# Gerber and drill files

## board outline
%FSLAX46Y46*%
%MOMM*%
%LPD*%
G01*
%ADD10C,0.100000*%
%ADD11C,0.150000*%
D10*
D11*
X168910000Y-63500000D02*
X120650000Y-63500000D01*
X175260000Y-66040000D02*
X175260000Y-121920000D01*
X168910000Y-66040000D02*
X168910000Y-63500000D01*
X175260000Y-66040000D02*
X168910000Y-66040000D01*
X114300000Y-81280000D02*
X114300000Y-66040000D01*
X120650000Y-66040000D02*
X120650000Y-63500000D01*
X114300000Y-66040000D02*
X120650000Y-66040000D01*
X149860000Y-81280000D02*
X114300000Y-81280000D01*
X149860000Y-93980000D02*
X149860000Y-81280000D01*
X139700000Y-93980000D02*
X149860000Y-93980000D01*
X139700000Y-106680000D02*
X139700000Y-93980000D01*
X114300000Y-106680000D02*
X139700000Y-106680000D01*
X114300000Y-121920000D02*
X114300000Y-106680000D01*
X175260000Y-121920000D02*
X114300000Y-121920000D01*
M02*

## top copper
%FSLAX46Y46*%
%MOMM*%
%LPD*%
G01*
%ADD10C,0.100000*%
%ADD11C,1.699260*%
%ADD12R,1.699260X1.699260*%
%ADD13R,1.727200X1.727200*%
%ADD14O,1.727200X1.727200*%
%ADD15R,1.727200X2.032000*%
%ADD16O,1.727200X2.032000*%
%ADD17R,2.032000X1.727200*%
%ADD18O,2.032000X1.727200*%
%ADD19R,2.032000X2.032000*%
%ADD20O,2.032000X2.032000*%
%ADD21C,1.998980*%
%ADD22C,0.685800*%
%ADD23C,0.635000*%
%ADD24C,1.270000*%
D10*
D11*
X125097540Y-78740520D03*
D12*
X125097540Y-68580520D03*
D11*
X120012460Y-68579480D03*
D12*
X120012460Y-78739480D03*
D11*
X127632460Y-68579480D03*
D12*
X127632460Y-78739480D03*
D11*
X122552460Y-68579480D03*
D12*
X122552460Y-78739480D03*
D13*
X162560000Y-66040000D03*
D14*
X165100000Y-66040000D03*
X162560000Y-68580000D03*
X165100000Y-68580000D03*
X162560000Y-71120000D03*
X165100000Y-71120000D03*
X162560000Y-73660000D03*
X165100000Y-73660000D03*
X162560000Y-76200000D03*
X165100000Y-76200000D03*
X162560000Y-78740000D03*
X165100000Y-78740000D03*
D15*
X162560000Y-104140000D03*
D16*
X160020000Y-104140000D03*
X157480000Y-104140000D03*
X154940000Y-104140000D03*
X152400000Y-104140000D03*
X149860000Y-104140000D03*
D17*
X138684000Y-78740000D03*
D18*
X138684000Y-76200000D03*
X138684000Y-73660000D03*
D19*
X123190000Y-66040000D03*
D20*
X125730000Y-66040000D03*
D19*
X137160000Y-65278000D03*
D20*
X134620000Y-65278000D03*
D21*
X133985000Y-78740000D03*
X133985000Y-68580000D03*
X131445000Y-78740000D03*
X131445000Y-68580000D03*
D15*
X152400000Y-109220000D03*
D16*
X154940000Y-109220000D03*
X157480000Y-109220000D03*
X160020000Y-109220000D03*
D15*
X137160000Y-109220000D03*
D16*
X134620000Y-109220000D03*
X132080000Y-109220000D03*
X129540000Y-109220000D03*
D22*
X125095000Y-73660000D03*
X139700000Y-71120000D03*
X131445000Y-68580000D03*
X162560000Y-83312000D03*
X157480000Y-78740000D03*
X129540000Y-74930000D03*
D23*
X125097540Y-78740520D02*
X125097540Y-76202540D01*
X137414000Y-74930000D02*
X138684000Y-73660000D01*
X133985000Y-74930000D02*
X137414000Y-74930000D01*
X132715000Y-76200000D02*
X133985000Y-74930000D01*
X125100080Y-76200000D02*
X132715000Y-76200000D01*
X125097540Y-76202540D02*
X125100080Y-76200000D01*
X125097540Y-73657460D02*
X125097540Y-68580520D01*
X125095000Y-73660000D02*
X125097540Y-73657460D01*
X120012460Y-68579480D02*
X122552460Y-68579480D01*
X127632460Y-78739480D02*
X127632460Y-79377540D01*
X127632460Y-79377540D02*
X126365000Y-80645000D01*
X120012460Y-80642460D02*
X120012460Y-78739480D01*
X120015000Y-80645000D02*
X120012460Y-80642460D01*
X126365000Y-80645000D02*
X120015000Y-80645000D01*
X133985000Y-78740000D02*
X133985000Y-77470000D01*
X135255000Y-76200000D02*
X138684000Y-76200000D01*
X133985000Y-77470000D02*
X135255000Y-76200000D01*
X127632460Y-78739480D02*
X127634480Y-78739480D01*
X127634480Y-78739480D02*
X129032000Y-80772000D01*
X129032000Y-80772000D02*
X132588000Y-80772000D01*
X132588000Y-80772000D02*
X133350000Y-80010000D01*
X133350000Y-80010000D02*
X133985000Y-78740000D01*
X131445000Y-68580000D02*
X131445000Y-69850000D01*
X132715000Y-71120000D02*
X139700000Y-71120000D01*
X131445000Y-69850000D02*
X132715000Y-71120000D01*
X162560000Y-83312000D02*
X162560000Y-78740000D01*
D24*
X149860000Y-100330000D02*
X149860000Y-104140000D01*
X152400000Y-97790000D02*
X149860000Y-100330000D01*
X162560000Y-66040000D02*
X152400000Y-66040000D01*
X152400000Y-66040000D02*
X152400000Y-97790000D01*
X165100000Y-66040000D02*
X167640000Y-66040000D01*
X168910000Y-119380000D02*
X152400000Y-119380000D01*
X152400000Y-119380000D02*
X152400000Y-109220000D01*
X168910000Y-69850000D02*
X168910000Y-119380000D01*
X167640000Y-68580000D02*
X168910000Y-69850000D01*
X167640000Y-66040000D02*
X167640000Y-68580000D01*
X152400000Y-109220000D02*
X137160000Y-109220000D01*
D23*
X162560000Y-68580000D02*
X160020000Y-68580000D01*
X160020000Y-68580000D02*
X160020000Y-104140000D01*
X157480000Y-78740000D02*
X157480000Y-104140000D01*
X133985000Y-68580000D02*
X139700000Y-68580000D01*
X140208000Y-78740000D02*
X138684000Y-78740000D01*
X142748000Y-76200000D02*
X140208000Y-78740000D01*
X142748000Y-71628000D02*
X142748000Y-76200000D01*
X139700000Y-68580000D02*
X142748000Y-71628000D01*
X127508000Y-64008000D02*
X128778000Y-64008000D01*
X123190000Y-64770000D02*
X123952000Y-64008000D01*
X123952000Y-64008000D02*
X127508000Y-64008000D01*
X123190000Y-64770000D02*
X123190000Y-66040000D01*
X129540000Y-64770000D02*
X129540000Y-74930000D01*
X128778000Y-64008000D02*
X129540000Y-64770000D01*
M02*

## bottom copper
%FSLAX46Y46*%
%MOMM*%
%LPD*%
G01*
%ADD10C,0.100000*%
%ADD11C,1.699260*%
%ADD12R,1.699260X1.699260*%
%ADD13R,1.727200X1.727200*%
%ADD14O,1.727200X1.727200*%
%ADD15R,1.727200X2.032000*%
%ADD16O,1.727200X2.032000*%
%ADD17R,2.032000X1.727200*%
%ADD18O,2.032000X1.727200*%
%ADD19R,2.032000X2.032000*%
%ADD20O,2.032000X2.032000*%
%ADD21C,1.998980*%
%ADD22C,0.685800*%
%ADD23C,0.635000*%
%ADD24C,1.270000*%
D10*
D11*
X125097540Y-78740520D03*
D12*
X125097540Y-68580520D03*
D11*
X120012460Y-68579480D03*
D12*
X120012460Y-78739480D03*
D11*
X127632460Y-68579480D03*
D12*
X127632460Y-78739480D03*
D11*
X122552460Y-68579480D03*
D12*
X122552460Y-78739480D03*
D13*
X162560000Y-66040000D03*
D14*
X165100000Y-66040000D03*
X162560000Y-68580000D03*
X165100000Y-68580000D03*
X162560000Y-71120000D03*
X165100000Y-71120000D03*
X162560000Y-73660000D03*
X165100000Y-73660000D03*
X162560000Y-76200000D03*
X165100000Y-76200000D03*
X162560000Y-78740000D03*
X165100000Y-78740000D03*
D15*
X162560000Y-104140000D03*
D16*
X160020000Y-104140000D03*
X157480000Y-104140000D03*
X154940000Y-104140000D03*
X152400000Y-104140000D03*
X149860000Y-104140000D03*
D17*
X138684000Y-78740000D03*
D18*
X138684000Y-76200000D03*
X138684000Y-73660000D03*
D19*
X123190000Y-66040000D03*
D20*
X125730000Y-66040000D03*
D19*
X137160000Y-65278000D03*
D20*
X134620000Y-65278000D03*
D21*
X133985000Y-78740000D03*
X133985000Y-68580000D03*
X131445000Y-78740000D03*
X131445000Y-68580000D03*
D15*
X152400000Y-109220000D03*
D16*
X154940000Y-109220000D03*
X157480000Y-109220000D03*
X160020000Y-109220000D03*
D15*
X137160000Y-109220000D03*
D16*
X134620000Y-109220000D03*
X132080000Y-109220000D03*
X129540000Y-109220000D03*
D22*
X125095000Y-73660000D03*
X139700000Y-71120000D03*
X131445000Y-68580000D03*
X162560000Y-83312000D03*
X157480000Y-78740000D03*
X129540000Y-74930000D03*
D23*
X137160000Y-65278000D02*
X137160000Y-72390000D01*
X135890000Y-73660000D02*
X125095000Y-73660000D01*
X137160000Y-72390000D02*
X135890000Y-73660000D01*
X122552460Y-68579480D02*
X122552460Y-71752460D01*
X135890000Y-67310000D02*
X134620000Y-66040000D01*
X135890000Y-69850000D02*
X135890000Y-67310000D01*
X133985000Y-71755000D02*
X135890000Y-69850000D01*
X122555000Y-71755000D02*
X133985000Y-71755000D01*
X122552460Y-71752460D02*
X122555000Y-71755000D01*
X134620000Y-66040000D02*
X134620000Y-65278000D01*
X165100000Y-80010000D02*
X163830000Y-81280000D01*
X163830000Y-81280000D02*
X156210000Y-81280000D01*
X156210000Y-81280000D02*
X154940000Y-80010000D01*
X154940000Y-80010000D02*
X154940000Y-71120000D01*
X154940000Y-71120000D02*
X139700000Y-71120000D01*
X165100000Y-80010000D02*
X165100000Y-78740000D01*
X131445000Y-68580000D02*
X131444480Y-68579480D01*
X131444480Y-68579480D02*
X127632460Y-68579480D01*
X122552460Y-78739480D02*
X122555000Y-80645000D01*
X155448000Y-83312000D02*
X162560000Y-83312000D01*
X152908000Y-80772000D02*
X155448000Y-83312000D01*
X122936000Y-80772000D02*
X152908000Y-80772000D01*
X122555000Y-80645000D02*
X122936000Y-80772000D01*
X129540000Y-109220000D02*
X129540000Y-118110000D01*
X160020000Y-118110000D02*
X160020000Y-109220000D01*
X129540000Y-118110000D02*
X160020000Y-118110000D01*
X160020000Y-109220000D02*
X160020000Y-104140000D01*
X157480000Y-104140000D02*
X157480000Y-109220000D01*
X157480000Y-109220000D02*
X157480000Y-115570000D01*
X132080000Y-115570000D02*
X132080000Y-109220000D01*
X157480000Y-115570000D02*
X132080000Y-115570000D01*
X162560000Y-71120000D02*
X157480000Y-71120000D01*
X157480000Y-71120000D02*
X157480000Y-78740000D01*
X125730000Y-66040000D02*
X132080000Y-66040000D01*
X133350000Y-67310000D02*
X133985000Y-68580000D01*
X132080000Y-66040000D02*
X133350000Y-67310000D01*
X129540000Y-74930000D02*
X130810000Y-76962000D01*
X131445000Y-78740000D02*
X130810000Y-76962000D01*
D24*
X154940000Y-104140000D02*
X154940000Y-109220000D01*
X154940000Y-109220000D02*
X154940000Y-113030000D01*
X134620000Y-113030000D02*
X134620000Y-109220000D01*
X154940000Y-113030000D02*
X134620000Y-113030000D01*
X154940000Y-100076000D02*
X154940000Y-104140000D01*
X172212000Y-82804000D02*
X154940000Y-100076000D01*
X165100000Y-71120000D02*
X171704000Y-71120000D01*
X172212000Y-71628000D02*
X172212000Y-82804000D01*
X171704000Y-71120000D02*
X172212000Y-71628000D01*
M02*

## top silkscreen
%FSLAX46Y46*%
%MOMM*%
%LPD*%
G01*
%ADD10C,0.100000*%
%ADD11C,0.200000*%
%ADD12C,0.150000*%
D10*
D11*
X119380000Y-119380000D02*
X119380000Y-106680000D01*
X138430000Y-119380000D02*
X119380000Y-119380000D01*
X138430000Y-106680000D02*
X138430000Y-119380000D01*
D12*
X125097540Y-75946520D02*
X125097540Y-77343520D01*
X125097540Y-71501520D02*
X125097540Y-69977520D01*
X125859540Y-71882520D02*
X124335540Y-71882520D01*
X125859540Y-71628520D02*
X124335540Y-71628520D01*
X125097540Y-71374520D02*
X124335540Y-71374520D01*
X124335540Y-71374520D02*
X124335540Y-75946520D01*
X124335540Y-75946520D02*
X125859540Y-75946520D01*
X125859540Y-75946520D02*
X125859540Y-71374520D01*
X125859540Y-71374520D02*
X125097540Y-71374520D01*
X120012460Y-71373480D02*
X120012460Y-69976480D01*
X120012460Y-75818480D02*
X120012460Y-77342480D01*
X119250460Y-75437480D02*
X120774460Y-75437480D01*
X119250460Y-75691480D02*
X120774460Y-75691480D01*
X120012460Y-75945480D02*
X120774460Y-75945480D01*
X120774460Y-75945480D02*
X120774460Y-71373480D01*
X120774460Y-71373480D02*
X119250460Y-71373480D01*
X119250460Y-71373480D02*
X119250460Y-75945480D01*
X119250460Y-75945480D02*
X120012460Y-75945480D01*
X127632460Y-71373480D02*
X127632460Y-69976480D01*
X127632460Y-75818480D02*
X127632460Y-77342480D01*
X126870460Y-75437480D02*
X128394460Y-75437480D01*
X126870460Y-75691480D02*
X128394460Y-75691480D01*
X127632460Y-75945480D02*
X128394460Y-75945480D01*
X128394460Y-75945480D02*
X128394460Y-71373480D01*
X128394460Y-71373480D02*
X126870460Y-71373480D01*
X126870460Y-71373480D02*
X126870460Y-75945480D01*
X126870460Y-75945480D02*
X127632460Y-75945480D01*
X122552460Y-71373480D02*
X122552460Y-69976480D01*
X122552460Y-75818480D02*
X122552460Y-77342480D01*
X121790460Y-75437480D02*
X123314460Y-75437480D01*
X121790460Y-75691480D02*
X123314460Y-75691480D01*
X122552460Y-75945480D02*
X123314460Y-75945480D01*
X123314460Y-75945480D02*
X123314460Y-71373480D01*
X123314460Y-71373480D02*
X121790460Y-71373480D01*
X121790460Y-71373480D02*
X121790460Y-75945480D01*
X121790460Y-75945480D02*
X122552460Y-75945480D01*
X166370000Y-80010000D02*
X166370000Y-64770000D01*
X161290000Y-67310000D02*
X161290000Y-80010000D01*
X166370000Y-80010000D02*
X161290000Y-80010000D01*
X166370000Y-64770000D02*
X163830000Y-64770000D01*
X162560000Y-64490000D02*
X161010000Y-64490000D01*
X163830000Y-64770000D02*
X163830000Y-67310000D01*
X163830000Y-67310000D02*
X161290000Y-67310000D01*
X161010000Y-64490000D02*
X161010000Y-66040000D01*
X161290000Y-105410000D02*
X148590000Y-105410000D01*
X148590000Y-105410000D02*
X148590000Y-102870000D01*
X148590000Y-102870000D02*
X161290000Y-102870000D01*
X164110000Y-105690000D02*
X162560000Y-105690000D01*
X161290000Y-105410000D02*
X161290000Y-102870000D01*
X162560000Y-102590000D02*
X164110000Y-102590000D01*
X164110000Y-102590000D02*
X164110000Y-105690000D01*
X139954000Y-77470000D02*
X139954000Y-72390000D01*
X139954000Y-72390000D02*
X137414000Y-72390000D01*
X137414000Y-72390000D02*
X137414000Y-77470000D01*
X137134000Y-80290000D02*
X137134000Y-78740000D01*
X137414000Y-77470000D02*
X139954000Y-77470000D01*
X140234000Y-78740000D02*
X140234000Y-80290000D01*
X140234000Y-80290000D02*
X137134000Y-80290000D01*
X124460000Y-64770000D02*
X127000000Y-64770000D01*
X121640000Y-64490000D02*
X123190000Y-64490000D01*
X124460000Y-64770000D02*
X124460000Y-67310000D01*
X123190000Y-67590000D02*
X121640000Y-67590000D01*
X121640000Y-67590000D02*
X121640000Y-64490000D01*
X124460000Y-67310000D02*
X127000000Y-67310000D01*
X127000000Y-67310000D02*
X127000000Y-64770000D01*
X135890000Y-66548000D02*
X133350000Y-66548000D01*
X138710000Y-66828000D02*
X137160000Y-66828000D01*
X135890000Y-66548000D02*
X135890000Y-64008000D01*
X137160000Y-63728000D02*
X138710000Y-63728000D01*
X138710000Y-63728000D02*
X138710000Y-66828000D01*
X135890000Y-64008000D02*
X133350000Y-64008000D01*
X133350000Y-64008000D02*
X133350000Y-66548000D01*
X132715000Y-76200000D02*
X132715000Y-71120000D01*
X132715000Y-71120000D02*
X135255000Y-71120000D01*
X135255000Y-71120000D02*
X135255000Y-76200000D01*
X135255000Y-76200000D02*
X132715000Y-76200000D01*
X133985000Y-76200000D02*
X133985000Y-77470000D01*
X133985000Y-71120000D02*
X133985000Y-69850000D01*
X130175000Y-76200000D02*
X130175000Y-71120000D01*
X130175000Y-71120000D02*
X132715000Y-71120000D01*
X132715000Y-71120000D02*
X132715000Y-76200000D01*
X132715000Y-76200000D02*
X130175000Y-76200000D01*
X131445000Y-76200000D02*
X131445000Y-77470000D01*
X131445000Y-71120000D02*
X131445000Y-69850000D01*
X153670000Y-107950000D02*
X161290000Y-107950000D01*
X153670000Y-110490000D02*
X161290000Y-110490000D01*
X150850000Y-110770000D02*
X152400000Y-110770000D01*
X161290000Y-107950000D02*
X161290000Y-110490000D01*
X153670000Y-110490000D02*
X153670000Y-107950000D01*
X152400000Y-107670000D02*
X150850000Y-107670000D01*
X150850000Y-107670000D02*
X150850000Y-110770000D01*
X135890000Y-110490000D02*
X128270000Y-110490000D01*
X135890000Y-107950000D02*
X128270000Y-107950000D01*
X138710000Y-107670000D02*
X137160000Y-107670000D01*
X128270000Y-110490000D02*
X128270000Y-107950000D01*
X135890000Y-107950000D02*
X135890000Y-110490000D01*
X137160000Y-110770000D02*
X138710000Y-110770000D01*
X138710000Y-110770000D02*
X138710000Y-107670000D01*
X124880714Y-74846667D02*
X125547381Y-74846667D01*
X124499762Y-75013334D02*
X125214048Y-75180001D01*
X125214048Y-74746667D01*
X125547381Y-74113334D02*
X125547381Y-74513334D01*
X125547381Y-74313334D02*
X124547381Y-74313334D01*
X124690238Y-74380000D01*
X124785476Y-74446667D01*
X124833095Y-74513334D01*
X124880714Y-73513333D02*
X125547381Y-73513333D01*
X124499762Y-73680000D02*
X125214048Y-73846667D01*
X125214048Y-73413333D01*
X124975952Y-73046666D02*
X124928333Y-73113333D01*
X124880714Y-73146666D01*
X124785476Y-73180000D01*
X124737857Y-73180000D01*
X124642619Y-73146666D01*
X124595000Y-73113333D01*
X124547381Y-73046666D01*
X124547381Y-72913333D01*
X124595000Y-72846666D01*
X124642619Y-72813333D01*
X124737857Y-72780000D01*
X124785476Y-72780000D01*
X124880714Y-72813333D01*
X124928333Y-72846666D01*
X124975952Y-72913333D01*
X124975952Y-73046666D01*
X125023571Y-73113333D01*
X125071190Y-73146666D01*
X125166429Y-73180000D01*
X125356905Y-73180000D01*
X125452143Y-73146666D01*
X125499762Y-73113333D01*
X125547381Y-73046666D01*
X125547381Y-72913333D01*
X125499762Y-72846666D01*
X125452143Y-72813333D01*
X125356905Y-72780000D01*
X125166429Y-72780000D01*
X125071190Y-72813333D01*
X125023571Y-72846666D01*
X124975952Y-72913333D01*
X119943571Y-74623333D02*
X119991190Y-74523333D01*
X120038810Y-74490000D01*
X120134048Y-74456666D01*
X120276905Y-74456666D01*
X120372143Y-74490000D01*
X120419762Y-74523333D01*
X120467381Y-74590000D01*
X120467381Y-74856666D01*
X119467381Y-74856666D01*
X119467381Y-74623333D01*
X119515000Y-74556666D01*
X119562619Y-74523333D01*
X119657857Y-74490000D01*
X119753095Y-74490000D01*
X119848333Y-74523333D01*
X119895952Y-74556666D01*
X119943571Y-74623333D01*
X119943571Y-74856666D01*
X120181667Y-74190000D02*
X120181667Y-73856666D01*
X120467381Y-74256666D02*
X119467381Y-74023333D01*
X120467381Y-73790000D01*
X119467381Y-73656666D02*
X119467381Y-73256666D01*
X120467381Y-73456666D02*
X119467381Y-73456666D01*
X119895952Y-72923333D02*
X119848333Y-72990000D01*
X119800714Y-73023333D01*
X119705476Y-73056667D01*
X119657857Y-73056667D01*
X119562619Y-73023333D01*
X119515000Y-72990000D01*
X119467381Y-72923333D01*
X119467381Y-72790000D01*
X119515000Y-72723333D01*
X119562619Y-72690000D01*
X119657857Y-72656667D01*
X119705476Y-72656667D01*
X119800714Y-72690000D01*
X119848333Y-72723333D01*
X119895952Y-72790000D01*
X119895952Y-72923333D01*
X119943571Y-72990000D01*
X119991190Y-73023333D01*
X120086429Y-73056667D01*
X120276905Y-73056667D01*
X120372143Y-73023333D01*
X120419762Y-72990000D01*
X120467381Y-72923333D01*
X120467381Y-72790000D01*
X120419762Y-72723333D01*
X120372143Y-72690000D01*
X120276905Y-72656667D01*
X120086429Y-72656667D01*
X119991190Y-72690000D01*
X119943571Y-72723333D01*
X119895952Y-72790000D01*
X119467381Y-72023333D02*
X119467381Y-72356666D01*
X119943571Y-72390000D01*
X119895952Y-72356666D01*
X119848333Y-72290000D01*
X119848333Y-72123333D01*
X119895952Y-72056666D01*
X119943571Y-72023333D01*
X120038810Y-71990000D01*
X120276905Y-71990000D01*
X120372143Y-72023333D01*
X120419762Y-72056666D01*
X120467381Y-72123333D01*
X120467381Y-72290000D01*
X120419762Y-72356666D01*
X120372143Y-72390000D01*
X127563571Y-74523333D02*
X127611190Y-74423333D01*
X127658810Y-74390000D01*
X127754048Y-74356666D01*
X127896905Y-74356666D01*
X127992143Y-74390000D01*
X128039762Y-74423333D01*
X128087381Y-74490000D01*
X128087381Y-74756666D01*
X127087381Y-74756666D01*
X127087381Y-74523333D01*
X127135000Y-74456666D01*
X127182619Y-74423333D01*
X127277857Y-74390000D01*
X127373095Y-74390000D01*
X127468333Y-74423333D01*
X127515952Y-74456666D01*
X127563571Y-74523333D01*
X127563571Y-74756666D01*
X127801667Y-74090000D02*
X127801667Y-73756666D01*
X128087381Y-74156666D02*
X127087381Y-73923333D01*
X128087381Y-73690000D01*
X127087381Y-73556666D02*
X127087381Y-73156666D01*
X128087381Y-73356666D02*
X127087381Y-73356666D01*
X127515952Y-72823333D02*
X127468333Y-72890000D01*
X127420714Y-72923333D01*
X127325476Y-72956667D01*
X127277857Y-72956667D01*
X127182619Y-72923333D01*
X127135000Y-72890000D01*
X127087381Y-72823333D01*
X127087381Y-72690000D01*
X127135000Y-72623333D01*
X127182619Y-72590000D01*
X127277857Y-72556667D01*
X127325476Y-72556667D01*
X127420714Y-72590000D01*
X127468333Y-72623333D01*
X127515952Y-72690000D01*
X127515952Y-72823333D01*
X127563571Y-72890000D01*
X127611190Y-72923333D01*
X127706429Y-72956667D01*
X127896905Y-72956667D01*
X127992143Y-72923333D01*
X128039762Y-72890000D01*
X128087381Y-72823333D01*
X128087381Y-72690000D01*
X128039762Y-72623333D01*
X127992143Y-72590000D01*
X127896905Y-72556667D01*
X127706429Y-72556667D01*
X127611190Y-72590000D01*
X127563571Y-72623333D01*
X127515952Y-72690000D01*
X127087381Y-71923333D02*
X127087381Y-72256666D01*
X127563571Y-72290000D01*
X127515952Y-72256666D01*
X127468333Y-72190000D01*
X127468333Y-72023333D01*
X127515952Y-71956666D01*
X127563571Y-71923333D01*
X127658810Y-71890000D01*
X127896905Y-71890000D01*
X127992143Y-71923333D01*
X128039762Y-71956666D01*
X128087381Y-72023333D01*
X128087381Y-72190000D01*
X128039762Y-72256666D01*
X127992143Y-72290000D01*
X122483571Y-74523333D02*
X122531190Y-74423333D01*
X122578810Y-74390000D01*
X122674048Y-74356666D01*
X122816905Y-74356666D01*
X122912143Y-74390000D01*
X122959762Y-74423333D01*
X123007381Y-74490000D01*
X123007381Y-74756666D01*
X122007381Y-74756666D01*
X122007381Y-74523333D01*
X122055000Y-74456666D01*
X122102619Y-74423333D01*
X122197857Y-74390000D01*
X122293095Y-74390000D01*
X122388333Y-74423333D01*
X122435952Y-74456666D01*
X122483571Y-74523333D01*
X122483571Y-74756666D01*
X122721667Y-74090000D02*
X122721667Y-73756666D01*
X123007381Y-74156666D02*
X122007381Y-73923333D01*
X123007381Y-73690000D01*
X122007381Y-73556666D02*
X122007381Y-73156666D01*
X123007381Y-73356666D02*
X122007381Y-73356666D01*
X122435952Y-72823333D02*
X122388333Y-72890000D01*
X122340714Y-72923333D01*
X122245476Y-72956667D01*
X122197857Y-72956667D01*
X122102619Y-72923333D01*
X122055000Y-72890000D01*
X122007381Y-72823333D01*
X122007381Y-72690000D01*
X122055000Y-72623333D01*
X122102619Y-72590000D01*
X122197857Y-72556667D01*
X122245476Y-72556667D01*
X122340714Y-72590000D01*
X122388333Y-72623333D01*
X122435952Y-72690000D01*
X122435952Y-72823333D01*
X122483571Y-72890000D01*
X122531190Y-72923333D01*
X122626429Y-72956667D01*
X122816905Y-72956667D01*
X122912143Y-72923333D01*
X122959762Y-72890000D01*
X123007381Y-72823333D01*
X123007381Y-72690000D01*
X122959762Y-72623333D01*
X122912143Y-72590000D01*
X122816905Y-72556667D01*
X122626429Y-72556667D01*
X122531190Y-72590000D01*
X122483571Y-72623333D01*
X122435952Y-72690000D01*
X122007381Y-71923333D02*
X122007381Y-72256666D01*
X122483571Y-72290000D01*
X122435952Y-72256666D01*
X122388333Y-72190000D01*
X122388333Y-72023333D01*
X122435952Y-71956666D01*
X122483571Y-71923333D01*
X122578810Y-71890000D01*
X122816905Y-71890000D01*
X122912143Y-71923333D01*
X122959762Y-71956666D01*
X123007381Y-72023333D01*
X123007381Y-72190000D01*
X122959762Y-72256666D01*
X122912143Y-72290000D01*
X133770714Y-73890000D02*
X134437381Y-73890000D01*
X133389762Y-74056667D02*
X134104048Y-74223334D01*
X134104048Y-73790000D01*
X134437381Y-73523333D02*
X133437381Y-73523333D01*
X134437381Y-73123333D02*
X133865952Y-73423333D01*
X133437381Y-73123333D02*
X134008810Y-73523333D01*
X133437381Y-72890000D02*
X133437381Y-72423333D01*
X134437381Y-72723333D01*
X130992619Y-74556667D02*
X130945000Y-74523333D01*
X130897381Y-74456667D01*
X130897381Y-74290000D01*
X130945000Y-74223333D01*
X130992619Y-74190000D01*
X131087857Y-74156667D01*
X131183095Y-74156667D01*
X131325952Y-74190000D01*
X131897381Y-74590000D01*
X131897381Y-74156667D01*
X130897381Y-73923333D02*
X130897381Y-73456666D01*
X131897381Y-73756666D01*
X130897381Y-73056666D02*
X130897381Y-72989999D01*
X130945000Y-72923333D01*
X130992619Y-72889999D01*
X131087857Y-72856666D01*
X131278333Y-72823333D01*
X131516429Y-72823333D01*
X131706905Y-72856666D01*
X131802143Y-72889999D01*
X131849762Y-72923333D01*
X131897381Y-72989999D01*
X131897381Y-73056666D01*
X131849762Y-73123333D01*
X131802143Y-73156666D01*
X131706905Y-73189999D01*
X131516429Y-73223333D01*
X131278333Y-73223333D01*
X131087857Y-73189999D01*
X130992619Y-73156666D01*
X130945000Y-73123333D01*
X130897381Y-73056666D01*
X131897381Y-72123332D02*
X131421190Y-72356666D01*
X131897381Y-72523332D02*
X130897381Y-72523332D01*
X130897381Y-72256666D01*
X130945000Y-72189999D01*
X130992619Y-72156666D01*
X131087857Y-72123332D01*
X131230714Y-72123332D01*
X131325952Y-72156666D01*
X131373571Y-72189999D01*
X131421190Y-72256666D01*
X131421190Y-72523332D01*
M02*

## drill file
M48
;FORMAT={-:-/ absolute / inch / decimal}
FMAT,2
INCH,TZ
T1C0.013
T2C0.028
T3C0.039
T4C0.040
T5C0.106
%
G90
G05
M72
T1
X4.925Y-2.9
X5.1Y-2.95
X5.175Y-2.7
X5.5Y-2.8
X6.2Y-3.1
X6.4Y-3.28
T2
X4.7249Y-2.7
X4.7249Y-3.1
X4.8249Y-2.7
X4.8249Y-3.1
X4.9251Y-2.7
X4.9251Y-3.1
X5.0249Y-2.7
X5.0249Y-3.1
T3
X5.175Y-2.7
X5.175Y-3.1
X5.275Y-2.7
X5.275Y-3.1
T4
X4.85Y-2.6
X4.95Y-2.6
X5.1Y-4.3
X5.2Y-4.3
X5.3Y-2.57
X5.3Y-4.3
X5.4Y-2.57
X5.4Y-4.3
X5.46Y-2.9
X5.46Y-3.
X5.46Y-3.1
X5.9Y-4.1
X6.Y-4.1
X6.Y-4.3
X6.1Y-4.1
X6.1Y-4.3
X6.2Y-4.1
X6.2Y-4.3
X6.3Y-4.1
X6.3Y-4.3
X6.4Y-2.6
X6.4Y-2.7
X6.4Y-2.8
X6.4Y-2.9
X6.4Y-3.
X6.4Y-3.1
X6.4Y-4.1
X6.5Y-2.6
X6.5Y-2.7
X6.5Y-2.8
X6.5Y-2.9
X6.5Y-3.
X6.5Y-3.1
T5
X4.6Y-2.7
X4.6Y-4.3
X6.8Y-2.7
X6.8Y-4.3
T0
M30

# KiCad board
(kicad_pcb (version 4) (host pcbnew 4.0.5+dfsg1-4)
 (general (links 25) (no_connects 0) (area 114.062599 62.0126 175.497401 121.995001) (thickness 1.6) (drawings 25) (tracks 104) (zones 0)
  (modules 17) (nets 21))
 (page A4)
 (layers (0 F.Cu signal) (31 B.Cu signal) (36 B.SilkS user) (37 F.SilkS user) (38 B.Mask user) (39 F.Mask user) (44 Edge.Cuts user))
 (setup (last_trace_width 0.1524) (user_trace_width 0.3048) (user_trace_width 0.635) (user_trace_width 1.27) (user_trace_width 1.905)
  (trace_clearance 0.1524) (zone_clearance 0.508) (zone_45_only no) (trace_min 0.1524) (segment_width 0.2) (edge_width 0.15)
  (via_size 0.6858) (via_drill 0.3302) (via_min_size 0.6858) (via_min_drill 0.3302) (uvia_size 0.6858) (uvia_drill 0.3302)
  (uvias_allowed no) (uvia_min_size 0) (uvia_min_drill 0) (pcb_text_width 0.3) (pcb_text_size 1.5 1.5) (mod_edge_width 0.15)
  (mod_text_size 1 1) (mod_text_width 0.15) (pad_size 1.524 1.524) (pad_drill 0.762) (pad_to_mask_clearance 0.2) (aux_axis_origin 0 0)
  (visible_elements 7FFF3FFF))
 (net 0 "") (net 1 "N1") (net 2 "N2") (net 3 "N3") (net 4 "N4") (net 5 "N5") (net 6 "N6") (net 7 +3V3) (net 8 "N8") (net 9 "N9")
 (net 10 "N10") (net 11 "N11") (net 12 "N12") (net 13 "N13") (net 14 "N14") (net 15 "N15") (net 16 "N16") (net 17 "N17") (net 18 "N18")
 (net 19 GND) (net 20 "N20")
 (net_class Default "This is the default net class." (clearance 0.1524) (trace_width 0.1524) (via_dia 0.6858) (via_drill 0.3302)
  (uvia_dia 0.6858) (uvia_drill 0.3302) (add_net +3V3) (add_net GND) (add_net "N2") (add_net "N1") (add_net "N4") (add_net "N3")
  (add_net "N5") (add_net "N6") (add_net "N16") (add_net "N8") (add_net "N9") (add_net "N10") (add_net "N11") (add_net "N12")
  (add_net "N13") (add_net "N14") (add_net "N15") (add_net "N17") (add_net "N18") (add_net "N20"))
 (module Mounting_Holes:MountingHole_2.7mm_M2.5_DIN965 (layer F.Cu) (at 172.72 68.58)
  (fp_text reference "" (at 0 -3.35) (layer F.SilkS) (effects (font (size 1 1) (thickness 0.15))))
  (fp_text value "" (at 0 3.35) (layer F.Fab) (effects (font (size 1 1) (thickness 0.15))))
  (pad 1 np_thru_hole circle (at 0 0) (size 2.7 2.7) (drill 2.7) (layers *.Cu *.Mask)))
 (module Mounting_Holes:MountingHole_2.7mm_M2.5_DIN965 (layer F.Cu) (at 116.84 68.58)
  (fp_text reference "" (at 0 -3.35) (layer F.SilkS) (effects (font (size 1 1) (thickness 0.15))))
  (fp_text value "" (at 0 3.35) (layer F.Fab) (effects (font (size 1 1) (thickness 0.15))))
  (pad 1 np_thru_hole circle (at 0 0) (size 2.7 2.7) (drill 2.7) (layers *.Cu *.Mask)))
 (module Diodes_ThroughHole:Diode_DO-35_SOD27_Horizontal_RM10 (layer F.Cu) (at 125.095 68.58 270)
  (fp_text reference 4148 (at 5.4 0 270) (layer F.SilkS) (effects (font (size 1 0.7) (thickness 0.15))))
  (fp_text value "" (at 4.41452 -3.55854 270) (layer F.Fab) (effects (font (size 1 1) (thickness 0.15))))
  (fp_line (start 7.36652 -0.00254) (end 8.76352 -0.00254) (layer F.SilkS) (width 0.15))
  (fp_line (start 2.92152 -0.00254) (end 1.39752 -0.00254) (layer F.SilkS) (width 0.15))
  (fp_line (start 3.30252 -0.76454) (end 3.30252 0.75946) (layer F.SilkS) (width 0.15))
  (fp_line (start 3.04852 -0.76454) (end 3.04852 0.75946) (layer F.SilkS) (width 0.15))
  (fp_line (start 2.79452 -0.00254) (end 2.79452 0.75946) (layer F.SilkS) (width 0.15))
  (fp_line (start 2.79452 0.75946) (end 7.36652 0.75946) (layer F.SilkS) (width 0.15))
  (fp_line (start 7.36652 0.75946) (end 7.36652 -0.76454) (layer F.SilkS) (width 0.15))
  (fp_line (start 7.36652 -0.76454) (end 2.79452 -0.76454) (layer F.SilkS) (width 0.15))
  (fp_line (start 2.79452 -0.76454) (end 2.79452 -0.00254) (layer F.SilkS) (width 0.15))
  (pad 2 thru_hole circle (at 10.16052 -0.00254 90) (size 1.69926 1.69926) (drill 0.70104) (layers *.Cu *.Mask) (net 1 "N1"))
  (pad 1 thru_hole rect (at 0.00052 -0.00254 90) (size 1.69926 1.69926) (drill 0.70104) (layers *.Cu *.Mask) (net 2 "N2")))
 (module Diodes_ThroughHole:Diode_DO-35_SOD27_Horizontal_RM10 (layer F.Cu) (at 120.015 78.74 90)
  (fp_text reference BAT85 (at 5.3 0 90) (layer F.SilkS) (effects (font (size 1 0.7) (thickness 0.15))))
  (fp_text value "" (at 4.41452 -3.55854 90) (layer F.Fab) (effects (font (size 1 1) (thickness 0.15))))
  (fp_line (start 7.36652 -0.00254) (end 8.76352 -0.00254) (layer F.SilkS) (width 0.15))
  (fp_line (start 2.92152 -0.00254) (end 1.39752 -0.00254) (layer F.SilkS) (width 0.15))
  (fp_line (start 3.30252 -0.76454) (end 3.30252 0.75946) (layer F.SilkS) (width 0.15))
  (fp_line (start 3.04852 -0.76454) (end 3.04852 0.75946) (layer F.SilkS) (width 0.15))
  (fp_line (start 2.79452 -0.00254) (end 2.79452 0.75946) (layer F.SilkS) (width 0.15))
  (fp_line (start 2.79452 0.75946) (end 7.36652 0.75946) (layer F.SilkS) (width 0.15))
  (fp_line (start 7.36652 0.75946) (end 7.36652 -0.76454) (layer F.SilkS) (width 0.15))
  (fp_line (start 7.36652 -0.76454) (end 2.79452 -0.76454) (layer F.SilkS) (width 0.15))
  (fp_line (start 2.79452 -0.76454) (end 2.79452 -0.00254) (layer F.SilkS) (width 0.15))
  (pad 2 thru_hole circle (at 10.16052 -0.00254 270) (size 1.69926 1.69926) (drill 0.70104) (layers *.Cu *.Mask) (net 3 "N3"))
  (pad 1 thru_hole rect (at 0.00052 -0.00254 270) (size 1.69926 1.69926) (drill 0.70104) (layers *.Cu *.Mask) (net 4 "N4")))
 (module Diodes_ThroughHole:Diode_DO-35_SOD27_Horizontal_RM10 (layer F.Cu) (at 127.635 78.74 90)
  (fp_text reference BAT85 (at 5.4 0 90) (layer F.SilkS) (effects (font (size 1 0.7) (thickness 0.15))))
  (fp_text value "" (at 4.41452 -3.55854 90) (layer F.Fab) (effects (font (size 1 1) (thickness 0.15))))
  (fp_line (start 7.36652 -0.00254) (end 8.76352 -0.00254) (layer F.SilkS) (width 0.15))
  (fp_line (start 2.92152 -0.00254) (end 1.39752 -0.00254) (layer F.SilkS) (width 0.15))
  (fp_line (start 3.30252 -0.76454) (end 3.30252 0.75946) (layer F.SilkS) (width 0.15))
  (fp_line (start 3.04852 -0.76454) (end 3.04852 0.75946) (layer F.SilkS) (width 0.15))
  (fp_line (start 2.79452 -0.00254) (end 2.79452 0.75946) (layer F.SilkS) (width 0.15))
  (fp_line (start 2.79452 0.75946) (end 7.36652 0.75946) (layer F.SilkS) (width 0.15))
  (fp_line (start 7.36652 0.75946) (end 7.36652 -0.76454) (layer F.SilkS) (width 0.15))
  (fp_line (start 7.36652 -0.76454) (end 2.79452 -0.76454) (layer F.SilkS) (width 0.15))
  (fp_line (start 2.79452 -0.76454) (end 2.79452 -0.00254) (layer F.SilkS) (width 0.15))
  (pad 2 thru_hole circle (at 10.16052 -0.00254 270) (size 1.69926 1.69926) (drill 0.70104) (layers *.Cu *.Mask) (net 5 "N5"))
  (pad 1 thru_hole rect (at 0.00052 -0.00254 270) (size 1.69926 1.69926) (drill 0.70104) (layers *.Cu *.Mask) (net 4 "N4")))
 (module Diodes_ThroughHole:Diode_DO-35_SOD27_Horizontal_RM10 (layer F.Cu) (at 122.555 78.74 90)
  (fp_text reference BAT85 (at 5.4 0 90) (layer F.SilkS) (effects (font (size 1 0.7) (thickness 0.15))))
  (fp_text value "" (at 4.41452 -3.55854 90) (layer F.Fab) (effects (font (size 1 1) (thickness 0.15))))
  (fp_line (start 7.36652 -0.00254) (end 8.76352 -0.00254) (layer F.SilkS) (width 0.15))
  (fp_line (start 2.92152 -0.00254) (end 1.39752 -0.00254) (layer F.SilkS) (width 0.15))
  (fp_line (start 3.30252 -0.76454) (end 3.30252 0.75946) (layer F.SilkS) (width 0.15))
  (fp_line (start 3.04852 -0.76454) (end 3.04852 0.75946) (layer F.SilkS) (width 0.15))
  (fp_line (start 2.79452 -0.00254) (end 2.79452 0.75946) (layer F.SilkS) (width 0.15))
  (fp_line (start 2.79452 0.75946) (end 7.36652 0.75946) (layer F.SilkS) (width 0.15))
  (fp_line (start 7.36652 0.75946) (end 7.36652 -0.76454) (layer F.SilkS) (width 0.15))
  (fp_line (start 7.36652 -0.76454) (end 2.79452 -0.76454) (layer F.SilkS) (width 0.15))
  (fp_line (start 2.79452 -0.76454) (end 2.79452 -0.00254) (layer F.SilkS) (width 0.15))
  (pad 2 thru_hole circle (at 10.16052 -0.00254 270) (size 1.69926 1.69926) (drill 0.70104) (layers *.Cu *.Mask) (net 3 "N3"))
  (pad 1 thru_hole rect (at 0.00052 -0.00254 270) (size 1.69926 1.69926) (drill 0.70104) (layers *.Cu *.Mask) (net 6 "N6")))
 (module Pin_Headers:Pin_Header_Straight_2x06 (layer F.Cu) (at 162.56 66.04)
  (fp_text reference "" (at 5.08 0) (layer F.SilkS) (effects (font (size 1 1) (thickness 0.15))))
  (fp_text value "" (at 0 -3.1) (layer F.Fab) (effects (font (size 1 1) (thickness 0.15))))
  (fp_line (start 3.81 13.97) (end 3.81 -1.27) (layer F.SilkS) (width 0.15))
  (fp_line (start -1.27 1.27) (end -1.27 13.97) (layer F.SilkS) (width 0.15))
  (fp_line (start 3.81 13.97) (end -1.27 13.97) (layer F.SilkS) (width 0.15))
  (fp_line (start 3.81 -1.27) (end 1.27 -1.27) (layer F.SilkS) (width 0.15))
  (fp_line (start 0 -1.55) (end -1.55 -1.55) (layer F.SilkS) (width 0.15))
  (fp_line (start 1.27 -1.27) (end 1.27 1.27) (layer F.SilkS) (width 0.15))
  (fp_line (start 1.27 1.27) (end -1.27 1.27) (layer F.SilkS) (width 0.15))
  (fp_line (start -1.55 -1.55) (end -1.55 0) (layer F.SilkS) (width 0.15))
  (pad 1 thru_hole rect (at 0 0) (size 1.7272 1.7272) (drill 1.016) (layers *.Cu *.Mask) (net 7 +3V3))
  (pad 2 thru_hole oval (at 2.54 0) (size 1.7272 1.7272) (drill 1.016) (layers *.Cu *.Mask) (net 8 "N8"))
  (pad 3 thru_hole oval (at 0 2.54) (size 1.7272 1.7272) (drill 1.016) (layers *.Cu *.Mask) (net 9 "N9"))
  (pad 4 thru_hole oval (at 2.54 2.54) (size 1.7272 1.7272) (drill 1.016) (layers *.Cu *.Mask) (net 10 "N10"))
  (pad 5 thru_hole oval (at 0 5.08) (size 1.7272 1.7272) (drill 1.016) (layers *.Cu *.Mask) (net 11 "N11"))
  (pad 6 thru_hole oval (at 2.54 5.08) (size 1.7272 1.7272) (drill 1.016) (layers *.Cu *.Mask) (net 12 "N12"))
  (pad 7 thru_hole oval (at 0 7.62) (size 1.7272 1.7272) (drill 1.016) (layers *.Cu *.Mask) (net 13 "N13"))
  (pad 8 thru_hole oval (at 2.54 7.62) (size 1.7272 1.7272) (drill 1.016) (layers *.Cu *.Mask) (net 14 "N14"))
  (pad 9 thru_hole oval (at 0 10.16) (size 1.7272 1.7272) (drill 1.016) (layers *.Cu *.Mask) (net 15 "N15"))
  (pad 10 thru_hole oval (at 2.54 10.16) (size 1.7272 1.7272) (drill 1.016) (layers *.Cu *.Mask) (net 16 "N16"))
  (pad 11 thru_hole oval (at 0 12.7) (size 1.7272 1.7272) (drill 1.016) (layers *.Cu *.Mask) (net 6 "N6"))
  (pad 12 thru_hole oval (at 2.54 12.7) (size 1.7272 1.7272) (drill 1.016) (layers *.Cu *.Mask) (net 5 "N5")))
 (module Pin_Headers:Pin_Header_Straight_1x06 (layer F.Cu) (at 162.56 104.14 270)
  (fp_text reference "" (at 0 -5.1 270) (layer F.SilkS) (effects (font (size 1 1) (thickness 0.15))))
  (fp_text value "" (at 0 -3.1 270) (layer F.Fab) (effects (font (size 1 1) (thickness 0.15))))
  (fp_line (start 1.27 1.27) (end 1.27 13.97) (layer F.SilkS) (width 0.15))
  (fp_line (start 1.27 13.97) (end -1.27 13.97) (layer F.SilkS) (width 0.15))
  (fp_line (start -1.27 13.97) (end -1.27 1.27) (layer F.SilkS) (width 0.15))
  (fp_line (start 1.55 -1.55) (end 1.55 0) (layer F.SilkS) (width 0.15))
  (fp_line (start 1.27 1.27) (end -1.27 1.27) (layer F.SilkS) (width 0.15))
  (fp_line (start -1.55 0) (end -1.55 -1.55) (layer F.SilkS) (width 0.15))
  (fp_line (start -1.55 -1.55) (end 1.55 -1.55) (layer F.SilkS) (width 0.15))
  (pad 1 thru_hole rect (at 0 0 270) (size 2.032 1.7272) (drill 1.016) (layers *.Cu *.Mask) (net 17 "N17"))
  (pad 2 thru_hole oval (at 0 2.54 270) (size 2.032 1.7272) (drill 1.016) (layers *.Cu *.Mask) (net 9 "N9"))
  (pad 3 thru_hole oval (at 0 5.08 270) (size 2.032 1.7272) (drill 1.016) (layers *.Cu *.Mask) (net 11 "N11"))
  (pad 4 thru_hole oval (at 0 7.62 270) (size 2.032 1.7272) (drill 1.016) (layers *.Cu *.Mask) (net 12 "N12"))
  (pad 5 thru_hole oval (at 0 10.16 270) (size 2.032 1.7272) (drill 1.016) (layers *.Cu *.Mask) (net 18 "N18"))
  (pad 6 thru_hole oval (at 0 12.7 270) (size 2.032 1.7272) (drill 1.016) (layers *.Cu *.Mask) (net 7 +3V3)))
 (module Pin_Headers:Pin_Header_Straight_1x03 (layer F.Cu) (at 138.684 78.74 180)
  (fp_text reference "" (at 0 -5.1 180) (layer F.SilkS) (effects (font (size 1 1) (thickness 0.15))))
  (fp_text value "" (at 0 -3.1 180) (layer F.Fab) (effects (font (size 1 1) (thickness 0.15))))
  (fp_line (start -1.27 1.27) (end -1.27 6.35) (layer F.SilkS) (width 0.15))
  (fp_line (start -1.27 6.35) (end 1.27 6.35) (layer F.SilkS) (width 0.15))
  (fp_line (start 1.27 6.35) (end 1.27 1.27) (layer F.SilkS) (width 0.15))
  (fp_line (start 1.55 -1.55) (end 1.55 0) (layer F.SilkS) (width 0.15))
  (fp_line (start 1.27 1.27) (end -1.27 1.27) (layer F.SilkS) (width 0.15))
  (fp_line (start -1.55 0) (end -1.55 -1.55) (layer F.SilkS) (width 0.15))
  (fp_line (start -1.55 -1.55) (end 1.55 -1.55) (layer F.SilkS) (width 0.15))
  (pad 1 thru_hole rect (at 0 0 180) (size 2.032 1.7272) (drill 1.016) (layers *.Cu *.Mask) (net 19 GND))
  (pad 2 thru_hole oval (at 0 2.54 180) (size 2.032 1.7272) (drill 1.016) (layers *.Cu *.Mask) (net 4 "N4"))
  (pad 3 thru_hole oval (at 0 5.08 180) (size 2.032 1.7272) (drill 1.016) (layers *.Cu *.Mask) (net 1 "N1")))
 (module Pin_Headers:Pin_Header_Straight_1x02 (layer F.Cu) (at 123.19 66.04 90)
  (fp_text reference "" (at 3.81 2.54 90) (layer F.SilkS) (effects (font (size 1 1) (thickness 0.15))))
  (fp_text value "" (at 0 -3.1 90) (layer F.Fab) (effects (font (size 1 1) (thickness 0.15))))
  (fp_line (start 1.27 1.27) (end 1.27 3.81) (layer F.SilkS) (width 0.15))
  (fp_line (start 1.55 -1.55) (end 1.55 0) (layer F.SilkS) (width 0.15))
  (fp_line (start 1.27 1.27) (end -1.27 1.27) (layer F.SilkS) (width 0.15))
  (fp_line (start -1.55 0) (end -1.55 -1.55) (layer F.SilkS) (width 0.15))
  (fp_line (start -1.55 -1.55) (end 1.55 -1.55) (layer F.SilkS) (width 0.15))
  (fp_line (start -1.27 1.27) (end -1.27 3.81) (layer F.SilkS) (width 0.15))
  (fp_line (start -1.27 3.81) (end 1.27 3.81) (layer F.SilkS) (width 0.15))
  (pad 1 thru_hole rect (at 0 0 90) (size 2.032 2.032) (drill 1.016) (layers *.Cu *.Mask) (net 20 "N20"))
  (pad 2 thru_hole oval (at 0 2.54 90) (size 2.032 2.032) (drill 1.016) (layers *.Cu *.Mask) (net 19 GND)))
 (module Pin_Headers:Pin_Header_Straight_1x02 (layer F.Cu) (at 137.16 65.278 270)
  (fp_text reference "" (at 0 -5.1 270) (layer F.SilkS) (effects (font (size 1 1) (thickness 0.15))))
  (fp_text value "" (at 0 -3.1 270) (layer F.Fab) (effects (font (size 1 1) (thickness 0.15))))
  (fp_line (start 1.27 1.27) (end 1.27 3.81) (layer F.SilkS) (width 0.15))
  (fp_line (start 1.55 -1.55) (end 1.55 0) (layer F.SilkS) (width 0.15))
  (fp_line (start 1.27 1.27) (end -1.27 1.27) (layer F.SilkS) (width 0.15))
  (fp_line (start -1.55 0) (end -1.55 -1.55) (layer F.SilkS) (width 0.15))
  (fp_line (start -1.55 -1.55) (end 1.55 -1.55) (layer F.SilkS) (width 0.15))
  (fp_line (start -1.27 1.27) (end -1.27 3.81) (layer F.SilkS) (width 0.15))
  (fp_line (start -1.27 3.81) (end 1.27 3.81) (layer F.SilkS) (width 0.15))
  (pad 1 thru_hole rect (at 0 0 270) (size 2.032 2.032) (drill 1.016) (layers *.Cu *.Mask) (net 2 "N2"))
  (pad 2 thru_hole oval (at 0 2.54 270) (size 2.032 2.032) (drill 1.016) (layers *.Cu *.Mask) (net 3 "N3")))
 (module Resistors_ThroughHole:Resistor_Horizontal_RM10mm (layer F.Cu) (at 133.985 78.74 90)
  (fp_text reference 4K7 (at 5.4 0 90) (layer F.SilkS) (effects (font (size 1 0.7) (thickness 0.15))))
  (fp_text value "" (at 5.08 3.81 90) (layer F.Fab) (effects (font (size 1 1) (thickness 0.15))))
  (fp_line (start 2.54 -1.27) (end 7.62 -1.27) (layer F.SilkS) (width 0.15))
  (fp_line (start 7.62 -1.27) (end 7.62 1.27) (layer F.SilkS) (width 0.15))
  (fp_line (start 7.62 1.27) (end 2.54 1.27) (layer F.SilkS) (width 0.15))
  (fp_line (start 2.54 1.27) (end 2.54 -1.27) (layer F.SilkS) (width 0.15))
  (fp_line (start 2.54 0) (end 1.27 0) (layer F.SilkS) (width 0.15))
  (fp_line (start 7.62 0) (end 8.89 0) (layer F.SilkS) (width 0.15))
  (pad 1 thru_hole circle (at 0 0 90) (size 1.99898 1.99898) (drill 1.00076) (layers *.Cu *.SilkS *.Mask) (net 4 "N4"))
  (pad 2 thru_hole circle (at 10.16 0 90) (size 1.99898 1.99898) (drill 1.00076) (layers *.Cu *.SilkS *.Mask) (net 19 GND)))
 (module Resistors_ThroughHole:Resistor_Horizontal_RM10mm (layer F.Cu) (at 131.445 78.74 90)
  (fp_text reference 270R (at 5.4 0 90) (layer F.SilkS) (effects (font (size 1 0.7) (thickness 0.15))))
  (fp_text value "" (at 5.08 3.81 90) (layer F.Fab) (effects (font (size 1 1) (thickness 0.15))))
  (fp_line (start 2.54 -1.27) (end 7.62 -1.27) (layer F.SilkS) (width 0.15))
  (fp_line (start 7.62 -1.27) (end 7.62 1.27) (layer F.SilkS) (width 0.15))
  (fp_line (start 7.62 1.27) (end 2.54 1.27) (layer F.SilkS) (width 0.15))
  (fp_line (start 2.54 1.27) (end 2.54 -1.27) (layer F.SilkS) (width 0.15))
  (fp_line (start 2.54 0) (end 1.27 0) (layer F.SilkS) (width 0.15))
  (fp_line (start 7.62 0) (end 8.89 0) (layer F.SilkS) (width 0.15))
  (pad 1 thru_hole circle (at 0 0 90) (size 1.99898 1.99898) (drill 1.00076) (layers *.Cu *.SilkS *.Mask) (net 20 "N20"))
  (pad 2 thru_hole circle (at 10.16 0 90) (size 1.99898 1.99898) (drill 1.00076) (layers *.Cu *.SilkS *.Mask) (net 5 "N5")))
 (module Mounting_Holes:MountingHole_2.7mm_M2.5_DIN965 (layer F.Cu) (at 172.72 109.22)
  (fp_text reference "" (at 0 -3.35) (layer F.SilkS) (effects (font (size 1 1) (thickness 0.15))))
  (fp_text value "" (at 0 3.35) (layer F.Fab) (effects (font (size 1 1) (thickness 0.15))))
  (pad 1 np_thru_hole circle (at 0 0) (size 2.7 2.7) (drill 2.7) (layers *.Cu *.Mask)))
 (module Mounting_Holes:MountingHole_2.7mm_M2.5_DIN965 (layer F.Cu) (at 116.84 109.22)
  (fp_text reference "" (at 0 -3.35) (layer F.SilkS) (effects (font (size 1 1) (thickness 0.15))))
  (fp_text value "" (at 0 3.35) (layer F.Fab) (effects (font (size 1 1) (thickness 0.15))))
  (pad 1 np_thru_hole circle (at 0 0) (size 2.7 2.7) (drill 2.7) (layers *.Cu *.Mask)))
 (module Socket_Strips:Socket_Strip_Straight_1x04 (layer F.Cu) (at 152.4 109.22)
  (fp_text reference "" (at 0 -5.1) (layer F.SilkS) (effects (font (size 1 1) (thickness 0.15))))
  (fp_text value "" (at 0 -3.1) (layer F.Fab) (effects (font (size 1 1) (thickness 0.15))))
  (fp_line (start 1.27 -1.27) (end 8.89 -1.27) (layer F.SilkS) (width 0.15))
  (fp_line (start 1.27 1.27) (end 8.89 1.27) (layer F.SilkS) (width 0.15))
  (fp_line (start -1.55 1.55) (end 0 1.55) (layer F.SilkS) (width 0.15))
  (fp_line (start 8.89 -1.27) (end 8.89 1.27) (layer F.SilkS) (width 0.15))
  (fp_line (start 1.27 1.27) (end 1.27 -1.27) (layer F.SilkS) (width 0.15))
  (fp_line (start 0 -1.55) (end -1.55 -1.55) (layer F.SilkS) (width 0.15))
  (fp_line (start -1.55 -1.55) (end -1.55 1.55) (layer F.SilkS) (width 0.15))
  (pad 1 thru_hole rect (at 0 0) (size 1.7272 2.032) (drill 1.016) (layers *.Cu *.Mask) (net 8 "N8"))
  (pad 2 thru_hole oval (at 2.54 0) (size 1.7272 2.032) (drill 1.016) (layers *.Cu *.Mask) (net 12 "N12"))
  (pad 3 thru_hole oval (at 5.08 0) (size 1.7272 2.032) (drill 1.016) (layers *.Cu *.Mask) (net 11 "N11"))
  (pad 4 thru_hole oval (at 7.62 0) (size 1.7272 2.032) (drill 1.016) (layers *.Cu *.Mask) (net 9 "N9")))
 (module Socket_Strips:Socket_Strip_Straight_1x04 (layer F.Cu) (at 137.16 109.22 180)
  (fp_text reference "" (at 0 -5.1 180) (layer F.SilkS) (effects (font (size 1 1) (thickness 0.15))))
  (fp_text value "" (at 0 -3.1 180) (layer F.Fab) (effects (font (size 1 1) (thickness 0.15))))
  (fp_line (start 1.27 -1.27) (end 8.89 -1.27) (layer F.SilkS) (width 0.15))
  (fp_line (start 1.27 1.27) (end 8.89 1.27) (layer F.SilkS) (width 0.15))
  (fp_line (start -1.55 1.55) (end 0 1.55) (layer F.SilkS) (width 0.15))
  (fp_line (start 8.89 -1.27) (end 8.89 1.27) (layer F.SilkS) (width 0.15))
  (fp_line (start 1.27 1.27) (end 1.27 -1.27) (layer F.SilkS) (width 0.15))
  (fp_line (start 0 -1.55) (end -1.55 -1.55) (layer F.SilkS) (width 0.15))
  (fp_line (start -1.55 -1.55) (end -1.55 1.55) (layer F.SilkS) (width 0.15))
  (pad 1 thru_hole rect (at 0 0 180) (size 1.7272 2.032) (drill 1.016) (layers *.Cu *.Mask) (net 8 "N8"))
  (pad 2 thru_hole oval (at 2.54 0 180) (size 1.7272 2.032) (drill 1.016) (layers *.Cu *.Mask) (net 12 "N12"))
  (pad 3 thru_hole oval (at 5.08 0 180) (size 1.7272 2.032) (drill 1.016) (layers *.Cu *.Mask) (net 11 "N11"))
  (pad 4 thru_hole oval (at 7.62 0 180) (size 1.7272 2.032) (drill 1.016) (layers *.Cu *.Mask) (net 9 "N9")))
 (gr_line (start 168.91 63.5) (end 120.65 63.5) (angle 90) (layer Edge.Cuts) (width 0.15))
 (gr_line (start 175.26 66.04) (end 175.26 121.92) (angle 90) (layer Edge.Cuts) (width 0.15))
 (gr_line (start 168.91 66.04) (end 168.91 63.5) (angle 90) (layer Edge.Cuts) (width 0.15))
 (gr_line (start 175.26 66.04) (end 168.91 66.04) (angle 90) (layer Edge.Cuts) (width 0.15))
 (gr_line (start 114.3 81.28) (end 114.3 66.04) (angle 90) (layer Edge.Cuts) (width 0.15))
 (gr_line (start 120.65 66.04) (end 120.65 63.5) (angle 90) (layer Edge.Cuts) (width 0.15))
 (gr_line (start 114.3 66.04) (end 120.65 66.04) (angle 90) (layer Edge.Cuts) (width 0.15))
 (gr_line (start 119.38 119.38) (end 119.38 106.68) (angle 90) (layer F.SilkS) (width 0.2))
 (gr_line (start 138.43 119.38) (end 119.38 119.38) (angle 90) (layer F.SilkS) (width 0.2))
 (gr_line (start 138.43 106.68) (end 138.43 119.38) (angle 90) (layer F.SilkS) (width 0.2))
 (gr_line (start 149.86 81.28) (end 114.3 81.28) (angle 90) (layer Edge.Cuts) (width 0.15))
 (gr_line (start 149.86 93.98) (end 149.86 81.28) (angle 90) (layer Edge.Cuts) (width 0.15))
 (gr_line (start 139.7 93.98) (end 149.86 93.98) (angle 90) (layer Edge.Cuts) (width 0.15))
 (gr_line (start 139.7 106.68) (end 139.7 93.98) (angle 90) (layer Edge.Cuts) (width 0.15))
 (gr_line (start 114.3 106.68) (end 139.7 106.68) (angle 90) (layer Edge.Cuts) (width 0.15))
 (gr_line (start 114.3 121.92) (end 114.3 106.68) (angle 90) (layer Edge.Cuts) (width 0.15))
 (gr_line (start 175.26 121.92) (end 114.3 121.92) (angle 90) (layer Edge.Cuts) (width 0.15))
 (segment (start 125.09754 78.74052) (end 125.09754 76.20254) (width 0.635) (layer F.Cu) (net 1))
 (segment (start 137.414 74.93) (end 138.684 73.66) (width 0.635) (layer F.Cu) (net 1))
 (segment (start 133.985 74.93) (end 137.414 74.93) (width 0.635) (layer F.Cu) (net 1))
 (segment (start 132.715 76.2) (end 133.985 74.93) (width 0.635) (layer F.Cu) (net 1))
 (segment (start 125.10008 76.2) (end 132.715 76.2) (width 0.635) (layer F.Cu) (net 1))
 (segment (start 125.09754 76.20254) (end 125.10008 76.2) (width 0.635) (layer F.Cu) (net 1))
 (segment (start 137.16 65.278) (end 137.16 72.39) (width 0.635) (layer B.Cu) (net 2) (status 10))
 (segment (start 125.09754 73.65746) (end 125.09754 68.58052) (width 0.635) (layer F.Cu) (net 2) (status 20))
 (segment (start 125.095 73.66) (end 125.09754 73.65746) (width 0.635) (layer F.Cu) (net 2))
 (via (at 125.095 73.66) (size 0.6858) (drill 0.3302) (layers F.Cu B.Cu) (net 2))
 (segment (start 135.89 73.66) (end 125.095 73.66) (width 0.635) (layer B.Cu) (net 2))
 (segment (start 137.16 72.39) (end 135.89 73.66) (width 0.635) (layer B.Cu) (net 2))
 (segment (start 122.55246 68.57948) (end 122.55246 71.75246) (width 0.635) (layer B.Cu) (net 3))
 (segment (start 135.89 67.31) (end 134.62 66.04) (width 0.635) (layer B.Cu) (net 3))
 (segment (start 135.89 69.85) (end 135.89 67.31) (width 0.635) (layer B.Cu) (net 3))
 (segment (start 133.985 71.755) (end 135.89 69.85) (width 0.635) (layer B.Cu) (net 3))
 (segment (start 122.555 71.755) (end 133.985 71.755) (width 0.635) (layer B.Cu) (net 3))
 (segment (start 122.55246 71.75246) (end 122.555 71.755) (width 0.635) (layer B.Cu) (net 3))
 (segment (start 134.62 66.04) (end 134.62 65.278) (width 0.635) (layer B.Cu) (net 3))
 (segment (start 120.01246 68.57948) (end 122.55246 68.57948) (width 0.635) (layer F.Cu) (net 3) (status 10))
 (segment (start 127.63246 78.73948) (end 127.63246 79.37754) (width 0.635) (layer F.Cu) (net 4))
 (segment (start 127.63246 79.37754) (end 126.365 80.645) (width 0.635) (layer F.Cu) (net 4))
 (segment (start 120.01246 80.64246) (end 120.01246 78.73948) (width 0.635) (layer F.Cu) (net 4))
 (segment (start 120.015 80.645) (end 120.01246 80.64246) (width 0.635) (layer F.Cu) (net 4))
 (segment (start 126.365 80.645) (end 120.015 80.645) (width 0.635) (layer F.Cu) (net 4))
 (segment (start 133.985 78.74) (end 133.985 77.47) (width 0.635) (layer F.Cu) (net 4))
 (segment (start 135.255 76.2) (end 138.684 76.2) (width 0.635) (layer F.Cu) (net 4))
 (segment (start 133.985 77.47) (end 135.255 76.2) (width 0.635) (layer F.Cu) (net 4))
 (segment (start 127.63246 78.73948) (end 127.63448 78.73948) (width 0.635) (layer F.Cu) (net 4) (status 30))
 (segment (start 127.63448 78.73948) (end 129.032 80.772) (width 0.635) (layer F.Cu) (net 4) (status 10))
 (segment (start 129.032 80.772) (end 132.588 80.772) (width 0.635) (layer F.Cu) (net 4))
 (segment (start 132.588 80.772) (end 133.35 80.01) (width 0.635) (layer F.Cu) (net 4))
 (segment (start 133.35 80.01) (end 133.985 78.74) (width 0.635) (layer F.Cu) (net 4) (status 20))
 (segment (start 131.445 68.58) (end 131.445 69.85) (width 0.635) (layer F.Cu) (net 5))
 (segment (start 165.1 80.01) (end 163.83 81.28) (width 0.635) (layer B.Cu) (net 5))
 (segment (start 163.83 81.28) (end 156.21 81.28) (width 0.635) (layer B.Cu) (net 5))
 (segment (start 156.21 81.28) (end 154.94 80.01) (width 0.635) (layer B.Cu) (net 5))
 (segment (start 154.94 80.01) (end 154.94 71.12) (width 0.635) (layer B.Cu) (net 5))
 (segment (start 154.94 71.12) (end 139.7 71.12) (width 0.635) (layer B.Cu) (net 5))
 (via (at 139.7 71.12) (size 0.6858) (drill 0.3302) (layers F.Cu B.Cu) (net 5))
 (segment (start 165.1 80.01) (end 165.1 78.74) (width 0.635) (layer B.Cu) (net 5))
 (segment (start 132.715 71.12) (end 139.7 71.12) (width 0.635) (layer F.Cu) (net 5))
 (segment (start 131.445 69.85) (end 132.715 71.12) (width 0.635) (layer F.Cu) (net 5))
 (via (at 131.445 68.58) (size 0.6858) (drill 0.3302) (layers F.Cu B.Cu) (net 5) (status 30))
 (segment (start 131.445 68.58) (end 131.44448 68.57948) (width 0.635) (layer B.Cu) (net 5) (status 30))
 (segment (start 131.44448 68.57948) (end 127.63246 68.57948) (width 0.635) (layer B.Cu) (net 5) (status 20))
 (segment (start 122.55246 78.73948) (end 122.555 80.645) (width 0.635) (layer B.Cu) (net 6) (status 10))
 (segment (start 162.56 83.312) (end 162.56 78.74) (width 0.635) (layer F.Cu) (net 6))
 (via (at 162.56 83.312) (size 0.6858) (drill 0.3302) (layers F.Cu B.Cu) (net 6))
 (segment (start 155.448 83.312) (end 162.56 83.312) (width 0.635) (layer B.Cu) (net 6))
 (segment (start 152.908 80.772) (end 155.448 83.312) (width 0.635) (layer B.Cu) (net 6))
 (segment (start 122.936 80.772) (end 152.908 80.772) (width 0.635) (layer B.Cu) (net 6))
 (segment (start 122.555 80.645) (end 122.936 80.772) (width 0.635) (layer B.Cu) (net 6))
 (segment (start 149.86 100.33) (end 149.86 104.14) (width 1.27) (layer F.Cu) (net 7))
 (segment (start 152.4 97.79) (end 149.86 100.33) (width 1.27) (layer F.Cu) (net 7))
 (segment (start 162.56 66.04) (end 152.4 66.04) (width 1.27) (layer F.Cu) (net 7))
 (segment (start 152.4 66.04) (end 152.4 97.79) (width 1.27) (layer F.Cu) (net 7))
 (segment (start 165.1 66.04) (end 167.64 66.04) (width 1.27) (layer F.Cu) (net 8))
 (segment (start 168.91 119.38) (end 152.4 119.38) (width 1.27) (layer F.Cu) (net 8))
 (segment (start 152.4 119.38) (end 152.4 109.22) (width 1.27) (layer F.Cu) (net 8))
 (segment (start 168.91 69.85) (end 168.91 119.38) (width 1.27) (layer F.Cu) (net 8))
 (segment (start 167.64 68.58) (end 168.91 69.85) (width 1.27) (layer F.Cu) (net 8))
 (segment (start 167.64 66.04) (end 167.64 68.58) (width 1.27) (layer F.Cu) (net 8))
 (segment (start 152.4 109.22) (end 137.16 109.22) (width 1.27) (layer F.Cu) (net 8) (status 20))
 (segment (start 129.54 109.22) (end 129.54 118.11) (width 0.635) (layer B.Cu) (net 9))
 (segment (start 160.02 118.11) (end 160.02 109.22) (width 0.635) (layer B.Cu) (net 9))
 (segment (start 129.54 118.11) (end 160.02 118.11) (width 0.635) (layer B.Cu) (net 9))
 (segment (start 160.02 109.22) (end 160.02 104.14) (width 0.635) (layer B.Cu) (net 9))
 (segment (start 162.56 68.58) (end 160.02 68.58) (width 0.635) (layer F.Cu) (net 9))
 (segment (start 160.02 68.58) (end 160.02 104.14) (width 0.635) (layer F.Cu) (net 9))
 (segment (start 157.48 104.14) (end 157.48 109.22) (width 0.635) (layer B.Cu) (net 11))
 (segment (start 157.48 109.22) (end 157.48 115.57) (width 0.635) (layer B.Cu) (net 11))
 (segment (start 132.08 115.57) (end 132.08 109.22) (width 0.635) (layer B.Cu) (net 11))
 (segment (start 157.48 115.57) (end 132.08 115.57) (width 0.635) (layer B.Cu) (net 11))
 (segment (start 162.56 71.12) (end 157.48 71.12) (width 0.635) (layer B.Cu) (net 11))
 (via (at 157.48 78.74) (size 0.6858) (drill 0.3302) (layers F.Cu B.Cu) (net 11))
 (segment (start 157.48 71.12) (end 157.48 78.74) (width 0.635) (layer B.Cu) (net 11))
 (segment (start 157.48 78.74) (end 157.48 104.14) (width 0.635) (layer F.Cu) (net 11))
 (segment (start 125.73 66.04) (end 132.08 66.04) (width 0.635) (layer B.Cu) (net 19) (status 10))
 (segment (start 133.35 67.31) (end 133.985 68.58) (width 0.635) (layer B.Cu) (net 19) (status 20))
 (segment (start 132.08 66.04) (end 133.35 67.31) (width 0.635) (layer B.Cu) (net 19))
 (segment (start 133.985 68.58) (end 139.7 68.58) (width 0.635) (layer F.Cu) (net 19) (status 10))
 (segment (start 140.208 78.74) (end 138.684 78.74) (width 0.635) (layer F.Cu) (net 19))
 (segment (start 142.748 76.2) (end 140.208 78.74) (width 0.635) (layer F.Cu) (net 19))
 (segment (start 142.748 71.628) (end 142.748 76.2) (width 0.635) (layer F.Cu) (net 19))
 (segment (start 139.7 68.58) (end 142.748 71.628) (width 0.635) (layer F.Cu) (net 19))
 (segment (start 127.508 64.008) (end 128.778 64.008) (width 0.635) (layer F.Cu) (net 20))
 (segment (start 123.19 64.77) (end 123.952 64.008) (width 0.635) (layer F.Cu) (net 20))
 (segment (start 123.952 64.008) (end 127.508 64.008) (width 0.635) (layer F.Cu) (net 20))
 (via (at 129.54 74.93) (size 0.6858) (drill 0.3302) (layers F.Cu B.Cu) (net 20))
 (segment (start 129.54 74.93) (end 130.81 76.962) (width 0.635) (layer B.Cu) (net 20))
 (segment (start 131.445 78.74) (end 130.81 76.962) (width 0.635) (layer B.Cu) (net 20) (status 20))
 (segment (start 123.19 64.77) (end 123.19 66.04) (width 0.635) (layer F.Cu) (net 20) (status 20))
 (segment (start 129.54 64.77) (end 129.54 74.93) (width 0.635) (layer F.Cu) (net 20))
 (segment (start 128.778 64.008) (end 129.54 64.77) (width 0.635) (layer F.Cu) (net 20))
 (segment (start 154.94 104.14) (end 154.94 109.22) (width 1.27) (layer B.Cu) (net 12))
 (segment (start 154.94 109.22) (end 154.94 113.03) (width 1.27) (layer B.Cu) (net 12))
 (segment (start 134.62 113.03) (end 134.62 109.22) (width 1.27) (layer B.Cu) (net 12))
 (segment (start 154.94 113.03) (end 134.62 113.03) (width 1.27) (layer B.Cu) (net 12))
 (segment (start 154.94 100.076) (end 154.94 104.14) (width 1.27) (layer B.Cu) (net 12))
 (segment (start 172.212 82.804) (end 154.94 100.076) (width 1.27) (layer B.Cu) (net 12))
 (segment (start 165.1 71.12) (end 171.704 71.12) (width 1.27) (layer B.Cu) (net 12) (status 10))
 (segment (start 172.212 71.628) (end 172.212 82.804) (width 1.27) (layer B.Cu) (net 12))
 (segment (start 171.704 71.12) (end 172.212 71.628) (width 1.27) (layer B.Cu) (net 12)))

